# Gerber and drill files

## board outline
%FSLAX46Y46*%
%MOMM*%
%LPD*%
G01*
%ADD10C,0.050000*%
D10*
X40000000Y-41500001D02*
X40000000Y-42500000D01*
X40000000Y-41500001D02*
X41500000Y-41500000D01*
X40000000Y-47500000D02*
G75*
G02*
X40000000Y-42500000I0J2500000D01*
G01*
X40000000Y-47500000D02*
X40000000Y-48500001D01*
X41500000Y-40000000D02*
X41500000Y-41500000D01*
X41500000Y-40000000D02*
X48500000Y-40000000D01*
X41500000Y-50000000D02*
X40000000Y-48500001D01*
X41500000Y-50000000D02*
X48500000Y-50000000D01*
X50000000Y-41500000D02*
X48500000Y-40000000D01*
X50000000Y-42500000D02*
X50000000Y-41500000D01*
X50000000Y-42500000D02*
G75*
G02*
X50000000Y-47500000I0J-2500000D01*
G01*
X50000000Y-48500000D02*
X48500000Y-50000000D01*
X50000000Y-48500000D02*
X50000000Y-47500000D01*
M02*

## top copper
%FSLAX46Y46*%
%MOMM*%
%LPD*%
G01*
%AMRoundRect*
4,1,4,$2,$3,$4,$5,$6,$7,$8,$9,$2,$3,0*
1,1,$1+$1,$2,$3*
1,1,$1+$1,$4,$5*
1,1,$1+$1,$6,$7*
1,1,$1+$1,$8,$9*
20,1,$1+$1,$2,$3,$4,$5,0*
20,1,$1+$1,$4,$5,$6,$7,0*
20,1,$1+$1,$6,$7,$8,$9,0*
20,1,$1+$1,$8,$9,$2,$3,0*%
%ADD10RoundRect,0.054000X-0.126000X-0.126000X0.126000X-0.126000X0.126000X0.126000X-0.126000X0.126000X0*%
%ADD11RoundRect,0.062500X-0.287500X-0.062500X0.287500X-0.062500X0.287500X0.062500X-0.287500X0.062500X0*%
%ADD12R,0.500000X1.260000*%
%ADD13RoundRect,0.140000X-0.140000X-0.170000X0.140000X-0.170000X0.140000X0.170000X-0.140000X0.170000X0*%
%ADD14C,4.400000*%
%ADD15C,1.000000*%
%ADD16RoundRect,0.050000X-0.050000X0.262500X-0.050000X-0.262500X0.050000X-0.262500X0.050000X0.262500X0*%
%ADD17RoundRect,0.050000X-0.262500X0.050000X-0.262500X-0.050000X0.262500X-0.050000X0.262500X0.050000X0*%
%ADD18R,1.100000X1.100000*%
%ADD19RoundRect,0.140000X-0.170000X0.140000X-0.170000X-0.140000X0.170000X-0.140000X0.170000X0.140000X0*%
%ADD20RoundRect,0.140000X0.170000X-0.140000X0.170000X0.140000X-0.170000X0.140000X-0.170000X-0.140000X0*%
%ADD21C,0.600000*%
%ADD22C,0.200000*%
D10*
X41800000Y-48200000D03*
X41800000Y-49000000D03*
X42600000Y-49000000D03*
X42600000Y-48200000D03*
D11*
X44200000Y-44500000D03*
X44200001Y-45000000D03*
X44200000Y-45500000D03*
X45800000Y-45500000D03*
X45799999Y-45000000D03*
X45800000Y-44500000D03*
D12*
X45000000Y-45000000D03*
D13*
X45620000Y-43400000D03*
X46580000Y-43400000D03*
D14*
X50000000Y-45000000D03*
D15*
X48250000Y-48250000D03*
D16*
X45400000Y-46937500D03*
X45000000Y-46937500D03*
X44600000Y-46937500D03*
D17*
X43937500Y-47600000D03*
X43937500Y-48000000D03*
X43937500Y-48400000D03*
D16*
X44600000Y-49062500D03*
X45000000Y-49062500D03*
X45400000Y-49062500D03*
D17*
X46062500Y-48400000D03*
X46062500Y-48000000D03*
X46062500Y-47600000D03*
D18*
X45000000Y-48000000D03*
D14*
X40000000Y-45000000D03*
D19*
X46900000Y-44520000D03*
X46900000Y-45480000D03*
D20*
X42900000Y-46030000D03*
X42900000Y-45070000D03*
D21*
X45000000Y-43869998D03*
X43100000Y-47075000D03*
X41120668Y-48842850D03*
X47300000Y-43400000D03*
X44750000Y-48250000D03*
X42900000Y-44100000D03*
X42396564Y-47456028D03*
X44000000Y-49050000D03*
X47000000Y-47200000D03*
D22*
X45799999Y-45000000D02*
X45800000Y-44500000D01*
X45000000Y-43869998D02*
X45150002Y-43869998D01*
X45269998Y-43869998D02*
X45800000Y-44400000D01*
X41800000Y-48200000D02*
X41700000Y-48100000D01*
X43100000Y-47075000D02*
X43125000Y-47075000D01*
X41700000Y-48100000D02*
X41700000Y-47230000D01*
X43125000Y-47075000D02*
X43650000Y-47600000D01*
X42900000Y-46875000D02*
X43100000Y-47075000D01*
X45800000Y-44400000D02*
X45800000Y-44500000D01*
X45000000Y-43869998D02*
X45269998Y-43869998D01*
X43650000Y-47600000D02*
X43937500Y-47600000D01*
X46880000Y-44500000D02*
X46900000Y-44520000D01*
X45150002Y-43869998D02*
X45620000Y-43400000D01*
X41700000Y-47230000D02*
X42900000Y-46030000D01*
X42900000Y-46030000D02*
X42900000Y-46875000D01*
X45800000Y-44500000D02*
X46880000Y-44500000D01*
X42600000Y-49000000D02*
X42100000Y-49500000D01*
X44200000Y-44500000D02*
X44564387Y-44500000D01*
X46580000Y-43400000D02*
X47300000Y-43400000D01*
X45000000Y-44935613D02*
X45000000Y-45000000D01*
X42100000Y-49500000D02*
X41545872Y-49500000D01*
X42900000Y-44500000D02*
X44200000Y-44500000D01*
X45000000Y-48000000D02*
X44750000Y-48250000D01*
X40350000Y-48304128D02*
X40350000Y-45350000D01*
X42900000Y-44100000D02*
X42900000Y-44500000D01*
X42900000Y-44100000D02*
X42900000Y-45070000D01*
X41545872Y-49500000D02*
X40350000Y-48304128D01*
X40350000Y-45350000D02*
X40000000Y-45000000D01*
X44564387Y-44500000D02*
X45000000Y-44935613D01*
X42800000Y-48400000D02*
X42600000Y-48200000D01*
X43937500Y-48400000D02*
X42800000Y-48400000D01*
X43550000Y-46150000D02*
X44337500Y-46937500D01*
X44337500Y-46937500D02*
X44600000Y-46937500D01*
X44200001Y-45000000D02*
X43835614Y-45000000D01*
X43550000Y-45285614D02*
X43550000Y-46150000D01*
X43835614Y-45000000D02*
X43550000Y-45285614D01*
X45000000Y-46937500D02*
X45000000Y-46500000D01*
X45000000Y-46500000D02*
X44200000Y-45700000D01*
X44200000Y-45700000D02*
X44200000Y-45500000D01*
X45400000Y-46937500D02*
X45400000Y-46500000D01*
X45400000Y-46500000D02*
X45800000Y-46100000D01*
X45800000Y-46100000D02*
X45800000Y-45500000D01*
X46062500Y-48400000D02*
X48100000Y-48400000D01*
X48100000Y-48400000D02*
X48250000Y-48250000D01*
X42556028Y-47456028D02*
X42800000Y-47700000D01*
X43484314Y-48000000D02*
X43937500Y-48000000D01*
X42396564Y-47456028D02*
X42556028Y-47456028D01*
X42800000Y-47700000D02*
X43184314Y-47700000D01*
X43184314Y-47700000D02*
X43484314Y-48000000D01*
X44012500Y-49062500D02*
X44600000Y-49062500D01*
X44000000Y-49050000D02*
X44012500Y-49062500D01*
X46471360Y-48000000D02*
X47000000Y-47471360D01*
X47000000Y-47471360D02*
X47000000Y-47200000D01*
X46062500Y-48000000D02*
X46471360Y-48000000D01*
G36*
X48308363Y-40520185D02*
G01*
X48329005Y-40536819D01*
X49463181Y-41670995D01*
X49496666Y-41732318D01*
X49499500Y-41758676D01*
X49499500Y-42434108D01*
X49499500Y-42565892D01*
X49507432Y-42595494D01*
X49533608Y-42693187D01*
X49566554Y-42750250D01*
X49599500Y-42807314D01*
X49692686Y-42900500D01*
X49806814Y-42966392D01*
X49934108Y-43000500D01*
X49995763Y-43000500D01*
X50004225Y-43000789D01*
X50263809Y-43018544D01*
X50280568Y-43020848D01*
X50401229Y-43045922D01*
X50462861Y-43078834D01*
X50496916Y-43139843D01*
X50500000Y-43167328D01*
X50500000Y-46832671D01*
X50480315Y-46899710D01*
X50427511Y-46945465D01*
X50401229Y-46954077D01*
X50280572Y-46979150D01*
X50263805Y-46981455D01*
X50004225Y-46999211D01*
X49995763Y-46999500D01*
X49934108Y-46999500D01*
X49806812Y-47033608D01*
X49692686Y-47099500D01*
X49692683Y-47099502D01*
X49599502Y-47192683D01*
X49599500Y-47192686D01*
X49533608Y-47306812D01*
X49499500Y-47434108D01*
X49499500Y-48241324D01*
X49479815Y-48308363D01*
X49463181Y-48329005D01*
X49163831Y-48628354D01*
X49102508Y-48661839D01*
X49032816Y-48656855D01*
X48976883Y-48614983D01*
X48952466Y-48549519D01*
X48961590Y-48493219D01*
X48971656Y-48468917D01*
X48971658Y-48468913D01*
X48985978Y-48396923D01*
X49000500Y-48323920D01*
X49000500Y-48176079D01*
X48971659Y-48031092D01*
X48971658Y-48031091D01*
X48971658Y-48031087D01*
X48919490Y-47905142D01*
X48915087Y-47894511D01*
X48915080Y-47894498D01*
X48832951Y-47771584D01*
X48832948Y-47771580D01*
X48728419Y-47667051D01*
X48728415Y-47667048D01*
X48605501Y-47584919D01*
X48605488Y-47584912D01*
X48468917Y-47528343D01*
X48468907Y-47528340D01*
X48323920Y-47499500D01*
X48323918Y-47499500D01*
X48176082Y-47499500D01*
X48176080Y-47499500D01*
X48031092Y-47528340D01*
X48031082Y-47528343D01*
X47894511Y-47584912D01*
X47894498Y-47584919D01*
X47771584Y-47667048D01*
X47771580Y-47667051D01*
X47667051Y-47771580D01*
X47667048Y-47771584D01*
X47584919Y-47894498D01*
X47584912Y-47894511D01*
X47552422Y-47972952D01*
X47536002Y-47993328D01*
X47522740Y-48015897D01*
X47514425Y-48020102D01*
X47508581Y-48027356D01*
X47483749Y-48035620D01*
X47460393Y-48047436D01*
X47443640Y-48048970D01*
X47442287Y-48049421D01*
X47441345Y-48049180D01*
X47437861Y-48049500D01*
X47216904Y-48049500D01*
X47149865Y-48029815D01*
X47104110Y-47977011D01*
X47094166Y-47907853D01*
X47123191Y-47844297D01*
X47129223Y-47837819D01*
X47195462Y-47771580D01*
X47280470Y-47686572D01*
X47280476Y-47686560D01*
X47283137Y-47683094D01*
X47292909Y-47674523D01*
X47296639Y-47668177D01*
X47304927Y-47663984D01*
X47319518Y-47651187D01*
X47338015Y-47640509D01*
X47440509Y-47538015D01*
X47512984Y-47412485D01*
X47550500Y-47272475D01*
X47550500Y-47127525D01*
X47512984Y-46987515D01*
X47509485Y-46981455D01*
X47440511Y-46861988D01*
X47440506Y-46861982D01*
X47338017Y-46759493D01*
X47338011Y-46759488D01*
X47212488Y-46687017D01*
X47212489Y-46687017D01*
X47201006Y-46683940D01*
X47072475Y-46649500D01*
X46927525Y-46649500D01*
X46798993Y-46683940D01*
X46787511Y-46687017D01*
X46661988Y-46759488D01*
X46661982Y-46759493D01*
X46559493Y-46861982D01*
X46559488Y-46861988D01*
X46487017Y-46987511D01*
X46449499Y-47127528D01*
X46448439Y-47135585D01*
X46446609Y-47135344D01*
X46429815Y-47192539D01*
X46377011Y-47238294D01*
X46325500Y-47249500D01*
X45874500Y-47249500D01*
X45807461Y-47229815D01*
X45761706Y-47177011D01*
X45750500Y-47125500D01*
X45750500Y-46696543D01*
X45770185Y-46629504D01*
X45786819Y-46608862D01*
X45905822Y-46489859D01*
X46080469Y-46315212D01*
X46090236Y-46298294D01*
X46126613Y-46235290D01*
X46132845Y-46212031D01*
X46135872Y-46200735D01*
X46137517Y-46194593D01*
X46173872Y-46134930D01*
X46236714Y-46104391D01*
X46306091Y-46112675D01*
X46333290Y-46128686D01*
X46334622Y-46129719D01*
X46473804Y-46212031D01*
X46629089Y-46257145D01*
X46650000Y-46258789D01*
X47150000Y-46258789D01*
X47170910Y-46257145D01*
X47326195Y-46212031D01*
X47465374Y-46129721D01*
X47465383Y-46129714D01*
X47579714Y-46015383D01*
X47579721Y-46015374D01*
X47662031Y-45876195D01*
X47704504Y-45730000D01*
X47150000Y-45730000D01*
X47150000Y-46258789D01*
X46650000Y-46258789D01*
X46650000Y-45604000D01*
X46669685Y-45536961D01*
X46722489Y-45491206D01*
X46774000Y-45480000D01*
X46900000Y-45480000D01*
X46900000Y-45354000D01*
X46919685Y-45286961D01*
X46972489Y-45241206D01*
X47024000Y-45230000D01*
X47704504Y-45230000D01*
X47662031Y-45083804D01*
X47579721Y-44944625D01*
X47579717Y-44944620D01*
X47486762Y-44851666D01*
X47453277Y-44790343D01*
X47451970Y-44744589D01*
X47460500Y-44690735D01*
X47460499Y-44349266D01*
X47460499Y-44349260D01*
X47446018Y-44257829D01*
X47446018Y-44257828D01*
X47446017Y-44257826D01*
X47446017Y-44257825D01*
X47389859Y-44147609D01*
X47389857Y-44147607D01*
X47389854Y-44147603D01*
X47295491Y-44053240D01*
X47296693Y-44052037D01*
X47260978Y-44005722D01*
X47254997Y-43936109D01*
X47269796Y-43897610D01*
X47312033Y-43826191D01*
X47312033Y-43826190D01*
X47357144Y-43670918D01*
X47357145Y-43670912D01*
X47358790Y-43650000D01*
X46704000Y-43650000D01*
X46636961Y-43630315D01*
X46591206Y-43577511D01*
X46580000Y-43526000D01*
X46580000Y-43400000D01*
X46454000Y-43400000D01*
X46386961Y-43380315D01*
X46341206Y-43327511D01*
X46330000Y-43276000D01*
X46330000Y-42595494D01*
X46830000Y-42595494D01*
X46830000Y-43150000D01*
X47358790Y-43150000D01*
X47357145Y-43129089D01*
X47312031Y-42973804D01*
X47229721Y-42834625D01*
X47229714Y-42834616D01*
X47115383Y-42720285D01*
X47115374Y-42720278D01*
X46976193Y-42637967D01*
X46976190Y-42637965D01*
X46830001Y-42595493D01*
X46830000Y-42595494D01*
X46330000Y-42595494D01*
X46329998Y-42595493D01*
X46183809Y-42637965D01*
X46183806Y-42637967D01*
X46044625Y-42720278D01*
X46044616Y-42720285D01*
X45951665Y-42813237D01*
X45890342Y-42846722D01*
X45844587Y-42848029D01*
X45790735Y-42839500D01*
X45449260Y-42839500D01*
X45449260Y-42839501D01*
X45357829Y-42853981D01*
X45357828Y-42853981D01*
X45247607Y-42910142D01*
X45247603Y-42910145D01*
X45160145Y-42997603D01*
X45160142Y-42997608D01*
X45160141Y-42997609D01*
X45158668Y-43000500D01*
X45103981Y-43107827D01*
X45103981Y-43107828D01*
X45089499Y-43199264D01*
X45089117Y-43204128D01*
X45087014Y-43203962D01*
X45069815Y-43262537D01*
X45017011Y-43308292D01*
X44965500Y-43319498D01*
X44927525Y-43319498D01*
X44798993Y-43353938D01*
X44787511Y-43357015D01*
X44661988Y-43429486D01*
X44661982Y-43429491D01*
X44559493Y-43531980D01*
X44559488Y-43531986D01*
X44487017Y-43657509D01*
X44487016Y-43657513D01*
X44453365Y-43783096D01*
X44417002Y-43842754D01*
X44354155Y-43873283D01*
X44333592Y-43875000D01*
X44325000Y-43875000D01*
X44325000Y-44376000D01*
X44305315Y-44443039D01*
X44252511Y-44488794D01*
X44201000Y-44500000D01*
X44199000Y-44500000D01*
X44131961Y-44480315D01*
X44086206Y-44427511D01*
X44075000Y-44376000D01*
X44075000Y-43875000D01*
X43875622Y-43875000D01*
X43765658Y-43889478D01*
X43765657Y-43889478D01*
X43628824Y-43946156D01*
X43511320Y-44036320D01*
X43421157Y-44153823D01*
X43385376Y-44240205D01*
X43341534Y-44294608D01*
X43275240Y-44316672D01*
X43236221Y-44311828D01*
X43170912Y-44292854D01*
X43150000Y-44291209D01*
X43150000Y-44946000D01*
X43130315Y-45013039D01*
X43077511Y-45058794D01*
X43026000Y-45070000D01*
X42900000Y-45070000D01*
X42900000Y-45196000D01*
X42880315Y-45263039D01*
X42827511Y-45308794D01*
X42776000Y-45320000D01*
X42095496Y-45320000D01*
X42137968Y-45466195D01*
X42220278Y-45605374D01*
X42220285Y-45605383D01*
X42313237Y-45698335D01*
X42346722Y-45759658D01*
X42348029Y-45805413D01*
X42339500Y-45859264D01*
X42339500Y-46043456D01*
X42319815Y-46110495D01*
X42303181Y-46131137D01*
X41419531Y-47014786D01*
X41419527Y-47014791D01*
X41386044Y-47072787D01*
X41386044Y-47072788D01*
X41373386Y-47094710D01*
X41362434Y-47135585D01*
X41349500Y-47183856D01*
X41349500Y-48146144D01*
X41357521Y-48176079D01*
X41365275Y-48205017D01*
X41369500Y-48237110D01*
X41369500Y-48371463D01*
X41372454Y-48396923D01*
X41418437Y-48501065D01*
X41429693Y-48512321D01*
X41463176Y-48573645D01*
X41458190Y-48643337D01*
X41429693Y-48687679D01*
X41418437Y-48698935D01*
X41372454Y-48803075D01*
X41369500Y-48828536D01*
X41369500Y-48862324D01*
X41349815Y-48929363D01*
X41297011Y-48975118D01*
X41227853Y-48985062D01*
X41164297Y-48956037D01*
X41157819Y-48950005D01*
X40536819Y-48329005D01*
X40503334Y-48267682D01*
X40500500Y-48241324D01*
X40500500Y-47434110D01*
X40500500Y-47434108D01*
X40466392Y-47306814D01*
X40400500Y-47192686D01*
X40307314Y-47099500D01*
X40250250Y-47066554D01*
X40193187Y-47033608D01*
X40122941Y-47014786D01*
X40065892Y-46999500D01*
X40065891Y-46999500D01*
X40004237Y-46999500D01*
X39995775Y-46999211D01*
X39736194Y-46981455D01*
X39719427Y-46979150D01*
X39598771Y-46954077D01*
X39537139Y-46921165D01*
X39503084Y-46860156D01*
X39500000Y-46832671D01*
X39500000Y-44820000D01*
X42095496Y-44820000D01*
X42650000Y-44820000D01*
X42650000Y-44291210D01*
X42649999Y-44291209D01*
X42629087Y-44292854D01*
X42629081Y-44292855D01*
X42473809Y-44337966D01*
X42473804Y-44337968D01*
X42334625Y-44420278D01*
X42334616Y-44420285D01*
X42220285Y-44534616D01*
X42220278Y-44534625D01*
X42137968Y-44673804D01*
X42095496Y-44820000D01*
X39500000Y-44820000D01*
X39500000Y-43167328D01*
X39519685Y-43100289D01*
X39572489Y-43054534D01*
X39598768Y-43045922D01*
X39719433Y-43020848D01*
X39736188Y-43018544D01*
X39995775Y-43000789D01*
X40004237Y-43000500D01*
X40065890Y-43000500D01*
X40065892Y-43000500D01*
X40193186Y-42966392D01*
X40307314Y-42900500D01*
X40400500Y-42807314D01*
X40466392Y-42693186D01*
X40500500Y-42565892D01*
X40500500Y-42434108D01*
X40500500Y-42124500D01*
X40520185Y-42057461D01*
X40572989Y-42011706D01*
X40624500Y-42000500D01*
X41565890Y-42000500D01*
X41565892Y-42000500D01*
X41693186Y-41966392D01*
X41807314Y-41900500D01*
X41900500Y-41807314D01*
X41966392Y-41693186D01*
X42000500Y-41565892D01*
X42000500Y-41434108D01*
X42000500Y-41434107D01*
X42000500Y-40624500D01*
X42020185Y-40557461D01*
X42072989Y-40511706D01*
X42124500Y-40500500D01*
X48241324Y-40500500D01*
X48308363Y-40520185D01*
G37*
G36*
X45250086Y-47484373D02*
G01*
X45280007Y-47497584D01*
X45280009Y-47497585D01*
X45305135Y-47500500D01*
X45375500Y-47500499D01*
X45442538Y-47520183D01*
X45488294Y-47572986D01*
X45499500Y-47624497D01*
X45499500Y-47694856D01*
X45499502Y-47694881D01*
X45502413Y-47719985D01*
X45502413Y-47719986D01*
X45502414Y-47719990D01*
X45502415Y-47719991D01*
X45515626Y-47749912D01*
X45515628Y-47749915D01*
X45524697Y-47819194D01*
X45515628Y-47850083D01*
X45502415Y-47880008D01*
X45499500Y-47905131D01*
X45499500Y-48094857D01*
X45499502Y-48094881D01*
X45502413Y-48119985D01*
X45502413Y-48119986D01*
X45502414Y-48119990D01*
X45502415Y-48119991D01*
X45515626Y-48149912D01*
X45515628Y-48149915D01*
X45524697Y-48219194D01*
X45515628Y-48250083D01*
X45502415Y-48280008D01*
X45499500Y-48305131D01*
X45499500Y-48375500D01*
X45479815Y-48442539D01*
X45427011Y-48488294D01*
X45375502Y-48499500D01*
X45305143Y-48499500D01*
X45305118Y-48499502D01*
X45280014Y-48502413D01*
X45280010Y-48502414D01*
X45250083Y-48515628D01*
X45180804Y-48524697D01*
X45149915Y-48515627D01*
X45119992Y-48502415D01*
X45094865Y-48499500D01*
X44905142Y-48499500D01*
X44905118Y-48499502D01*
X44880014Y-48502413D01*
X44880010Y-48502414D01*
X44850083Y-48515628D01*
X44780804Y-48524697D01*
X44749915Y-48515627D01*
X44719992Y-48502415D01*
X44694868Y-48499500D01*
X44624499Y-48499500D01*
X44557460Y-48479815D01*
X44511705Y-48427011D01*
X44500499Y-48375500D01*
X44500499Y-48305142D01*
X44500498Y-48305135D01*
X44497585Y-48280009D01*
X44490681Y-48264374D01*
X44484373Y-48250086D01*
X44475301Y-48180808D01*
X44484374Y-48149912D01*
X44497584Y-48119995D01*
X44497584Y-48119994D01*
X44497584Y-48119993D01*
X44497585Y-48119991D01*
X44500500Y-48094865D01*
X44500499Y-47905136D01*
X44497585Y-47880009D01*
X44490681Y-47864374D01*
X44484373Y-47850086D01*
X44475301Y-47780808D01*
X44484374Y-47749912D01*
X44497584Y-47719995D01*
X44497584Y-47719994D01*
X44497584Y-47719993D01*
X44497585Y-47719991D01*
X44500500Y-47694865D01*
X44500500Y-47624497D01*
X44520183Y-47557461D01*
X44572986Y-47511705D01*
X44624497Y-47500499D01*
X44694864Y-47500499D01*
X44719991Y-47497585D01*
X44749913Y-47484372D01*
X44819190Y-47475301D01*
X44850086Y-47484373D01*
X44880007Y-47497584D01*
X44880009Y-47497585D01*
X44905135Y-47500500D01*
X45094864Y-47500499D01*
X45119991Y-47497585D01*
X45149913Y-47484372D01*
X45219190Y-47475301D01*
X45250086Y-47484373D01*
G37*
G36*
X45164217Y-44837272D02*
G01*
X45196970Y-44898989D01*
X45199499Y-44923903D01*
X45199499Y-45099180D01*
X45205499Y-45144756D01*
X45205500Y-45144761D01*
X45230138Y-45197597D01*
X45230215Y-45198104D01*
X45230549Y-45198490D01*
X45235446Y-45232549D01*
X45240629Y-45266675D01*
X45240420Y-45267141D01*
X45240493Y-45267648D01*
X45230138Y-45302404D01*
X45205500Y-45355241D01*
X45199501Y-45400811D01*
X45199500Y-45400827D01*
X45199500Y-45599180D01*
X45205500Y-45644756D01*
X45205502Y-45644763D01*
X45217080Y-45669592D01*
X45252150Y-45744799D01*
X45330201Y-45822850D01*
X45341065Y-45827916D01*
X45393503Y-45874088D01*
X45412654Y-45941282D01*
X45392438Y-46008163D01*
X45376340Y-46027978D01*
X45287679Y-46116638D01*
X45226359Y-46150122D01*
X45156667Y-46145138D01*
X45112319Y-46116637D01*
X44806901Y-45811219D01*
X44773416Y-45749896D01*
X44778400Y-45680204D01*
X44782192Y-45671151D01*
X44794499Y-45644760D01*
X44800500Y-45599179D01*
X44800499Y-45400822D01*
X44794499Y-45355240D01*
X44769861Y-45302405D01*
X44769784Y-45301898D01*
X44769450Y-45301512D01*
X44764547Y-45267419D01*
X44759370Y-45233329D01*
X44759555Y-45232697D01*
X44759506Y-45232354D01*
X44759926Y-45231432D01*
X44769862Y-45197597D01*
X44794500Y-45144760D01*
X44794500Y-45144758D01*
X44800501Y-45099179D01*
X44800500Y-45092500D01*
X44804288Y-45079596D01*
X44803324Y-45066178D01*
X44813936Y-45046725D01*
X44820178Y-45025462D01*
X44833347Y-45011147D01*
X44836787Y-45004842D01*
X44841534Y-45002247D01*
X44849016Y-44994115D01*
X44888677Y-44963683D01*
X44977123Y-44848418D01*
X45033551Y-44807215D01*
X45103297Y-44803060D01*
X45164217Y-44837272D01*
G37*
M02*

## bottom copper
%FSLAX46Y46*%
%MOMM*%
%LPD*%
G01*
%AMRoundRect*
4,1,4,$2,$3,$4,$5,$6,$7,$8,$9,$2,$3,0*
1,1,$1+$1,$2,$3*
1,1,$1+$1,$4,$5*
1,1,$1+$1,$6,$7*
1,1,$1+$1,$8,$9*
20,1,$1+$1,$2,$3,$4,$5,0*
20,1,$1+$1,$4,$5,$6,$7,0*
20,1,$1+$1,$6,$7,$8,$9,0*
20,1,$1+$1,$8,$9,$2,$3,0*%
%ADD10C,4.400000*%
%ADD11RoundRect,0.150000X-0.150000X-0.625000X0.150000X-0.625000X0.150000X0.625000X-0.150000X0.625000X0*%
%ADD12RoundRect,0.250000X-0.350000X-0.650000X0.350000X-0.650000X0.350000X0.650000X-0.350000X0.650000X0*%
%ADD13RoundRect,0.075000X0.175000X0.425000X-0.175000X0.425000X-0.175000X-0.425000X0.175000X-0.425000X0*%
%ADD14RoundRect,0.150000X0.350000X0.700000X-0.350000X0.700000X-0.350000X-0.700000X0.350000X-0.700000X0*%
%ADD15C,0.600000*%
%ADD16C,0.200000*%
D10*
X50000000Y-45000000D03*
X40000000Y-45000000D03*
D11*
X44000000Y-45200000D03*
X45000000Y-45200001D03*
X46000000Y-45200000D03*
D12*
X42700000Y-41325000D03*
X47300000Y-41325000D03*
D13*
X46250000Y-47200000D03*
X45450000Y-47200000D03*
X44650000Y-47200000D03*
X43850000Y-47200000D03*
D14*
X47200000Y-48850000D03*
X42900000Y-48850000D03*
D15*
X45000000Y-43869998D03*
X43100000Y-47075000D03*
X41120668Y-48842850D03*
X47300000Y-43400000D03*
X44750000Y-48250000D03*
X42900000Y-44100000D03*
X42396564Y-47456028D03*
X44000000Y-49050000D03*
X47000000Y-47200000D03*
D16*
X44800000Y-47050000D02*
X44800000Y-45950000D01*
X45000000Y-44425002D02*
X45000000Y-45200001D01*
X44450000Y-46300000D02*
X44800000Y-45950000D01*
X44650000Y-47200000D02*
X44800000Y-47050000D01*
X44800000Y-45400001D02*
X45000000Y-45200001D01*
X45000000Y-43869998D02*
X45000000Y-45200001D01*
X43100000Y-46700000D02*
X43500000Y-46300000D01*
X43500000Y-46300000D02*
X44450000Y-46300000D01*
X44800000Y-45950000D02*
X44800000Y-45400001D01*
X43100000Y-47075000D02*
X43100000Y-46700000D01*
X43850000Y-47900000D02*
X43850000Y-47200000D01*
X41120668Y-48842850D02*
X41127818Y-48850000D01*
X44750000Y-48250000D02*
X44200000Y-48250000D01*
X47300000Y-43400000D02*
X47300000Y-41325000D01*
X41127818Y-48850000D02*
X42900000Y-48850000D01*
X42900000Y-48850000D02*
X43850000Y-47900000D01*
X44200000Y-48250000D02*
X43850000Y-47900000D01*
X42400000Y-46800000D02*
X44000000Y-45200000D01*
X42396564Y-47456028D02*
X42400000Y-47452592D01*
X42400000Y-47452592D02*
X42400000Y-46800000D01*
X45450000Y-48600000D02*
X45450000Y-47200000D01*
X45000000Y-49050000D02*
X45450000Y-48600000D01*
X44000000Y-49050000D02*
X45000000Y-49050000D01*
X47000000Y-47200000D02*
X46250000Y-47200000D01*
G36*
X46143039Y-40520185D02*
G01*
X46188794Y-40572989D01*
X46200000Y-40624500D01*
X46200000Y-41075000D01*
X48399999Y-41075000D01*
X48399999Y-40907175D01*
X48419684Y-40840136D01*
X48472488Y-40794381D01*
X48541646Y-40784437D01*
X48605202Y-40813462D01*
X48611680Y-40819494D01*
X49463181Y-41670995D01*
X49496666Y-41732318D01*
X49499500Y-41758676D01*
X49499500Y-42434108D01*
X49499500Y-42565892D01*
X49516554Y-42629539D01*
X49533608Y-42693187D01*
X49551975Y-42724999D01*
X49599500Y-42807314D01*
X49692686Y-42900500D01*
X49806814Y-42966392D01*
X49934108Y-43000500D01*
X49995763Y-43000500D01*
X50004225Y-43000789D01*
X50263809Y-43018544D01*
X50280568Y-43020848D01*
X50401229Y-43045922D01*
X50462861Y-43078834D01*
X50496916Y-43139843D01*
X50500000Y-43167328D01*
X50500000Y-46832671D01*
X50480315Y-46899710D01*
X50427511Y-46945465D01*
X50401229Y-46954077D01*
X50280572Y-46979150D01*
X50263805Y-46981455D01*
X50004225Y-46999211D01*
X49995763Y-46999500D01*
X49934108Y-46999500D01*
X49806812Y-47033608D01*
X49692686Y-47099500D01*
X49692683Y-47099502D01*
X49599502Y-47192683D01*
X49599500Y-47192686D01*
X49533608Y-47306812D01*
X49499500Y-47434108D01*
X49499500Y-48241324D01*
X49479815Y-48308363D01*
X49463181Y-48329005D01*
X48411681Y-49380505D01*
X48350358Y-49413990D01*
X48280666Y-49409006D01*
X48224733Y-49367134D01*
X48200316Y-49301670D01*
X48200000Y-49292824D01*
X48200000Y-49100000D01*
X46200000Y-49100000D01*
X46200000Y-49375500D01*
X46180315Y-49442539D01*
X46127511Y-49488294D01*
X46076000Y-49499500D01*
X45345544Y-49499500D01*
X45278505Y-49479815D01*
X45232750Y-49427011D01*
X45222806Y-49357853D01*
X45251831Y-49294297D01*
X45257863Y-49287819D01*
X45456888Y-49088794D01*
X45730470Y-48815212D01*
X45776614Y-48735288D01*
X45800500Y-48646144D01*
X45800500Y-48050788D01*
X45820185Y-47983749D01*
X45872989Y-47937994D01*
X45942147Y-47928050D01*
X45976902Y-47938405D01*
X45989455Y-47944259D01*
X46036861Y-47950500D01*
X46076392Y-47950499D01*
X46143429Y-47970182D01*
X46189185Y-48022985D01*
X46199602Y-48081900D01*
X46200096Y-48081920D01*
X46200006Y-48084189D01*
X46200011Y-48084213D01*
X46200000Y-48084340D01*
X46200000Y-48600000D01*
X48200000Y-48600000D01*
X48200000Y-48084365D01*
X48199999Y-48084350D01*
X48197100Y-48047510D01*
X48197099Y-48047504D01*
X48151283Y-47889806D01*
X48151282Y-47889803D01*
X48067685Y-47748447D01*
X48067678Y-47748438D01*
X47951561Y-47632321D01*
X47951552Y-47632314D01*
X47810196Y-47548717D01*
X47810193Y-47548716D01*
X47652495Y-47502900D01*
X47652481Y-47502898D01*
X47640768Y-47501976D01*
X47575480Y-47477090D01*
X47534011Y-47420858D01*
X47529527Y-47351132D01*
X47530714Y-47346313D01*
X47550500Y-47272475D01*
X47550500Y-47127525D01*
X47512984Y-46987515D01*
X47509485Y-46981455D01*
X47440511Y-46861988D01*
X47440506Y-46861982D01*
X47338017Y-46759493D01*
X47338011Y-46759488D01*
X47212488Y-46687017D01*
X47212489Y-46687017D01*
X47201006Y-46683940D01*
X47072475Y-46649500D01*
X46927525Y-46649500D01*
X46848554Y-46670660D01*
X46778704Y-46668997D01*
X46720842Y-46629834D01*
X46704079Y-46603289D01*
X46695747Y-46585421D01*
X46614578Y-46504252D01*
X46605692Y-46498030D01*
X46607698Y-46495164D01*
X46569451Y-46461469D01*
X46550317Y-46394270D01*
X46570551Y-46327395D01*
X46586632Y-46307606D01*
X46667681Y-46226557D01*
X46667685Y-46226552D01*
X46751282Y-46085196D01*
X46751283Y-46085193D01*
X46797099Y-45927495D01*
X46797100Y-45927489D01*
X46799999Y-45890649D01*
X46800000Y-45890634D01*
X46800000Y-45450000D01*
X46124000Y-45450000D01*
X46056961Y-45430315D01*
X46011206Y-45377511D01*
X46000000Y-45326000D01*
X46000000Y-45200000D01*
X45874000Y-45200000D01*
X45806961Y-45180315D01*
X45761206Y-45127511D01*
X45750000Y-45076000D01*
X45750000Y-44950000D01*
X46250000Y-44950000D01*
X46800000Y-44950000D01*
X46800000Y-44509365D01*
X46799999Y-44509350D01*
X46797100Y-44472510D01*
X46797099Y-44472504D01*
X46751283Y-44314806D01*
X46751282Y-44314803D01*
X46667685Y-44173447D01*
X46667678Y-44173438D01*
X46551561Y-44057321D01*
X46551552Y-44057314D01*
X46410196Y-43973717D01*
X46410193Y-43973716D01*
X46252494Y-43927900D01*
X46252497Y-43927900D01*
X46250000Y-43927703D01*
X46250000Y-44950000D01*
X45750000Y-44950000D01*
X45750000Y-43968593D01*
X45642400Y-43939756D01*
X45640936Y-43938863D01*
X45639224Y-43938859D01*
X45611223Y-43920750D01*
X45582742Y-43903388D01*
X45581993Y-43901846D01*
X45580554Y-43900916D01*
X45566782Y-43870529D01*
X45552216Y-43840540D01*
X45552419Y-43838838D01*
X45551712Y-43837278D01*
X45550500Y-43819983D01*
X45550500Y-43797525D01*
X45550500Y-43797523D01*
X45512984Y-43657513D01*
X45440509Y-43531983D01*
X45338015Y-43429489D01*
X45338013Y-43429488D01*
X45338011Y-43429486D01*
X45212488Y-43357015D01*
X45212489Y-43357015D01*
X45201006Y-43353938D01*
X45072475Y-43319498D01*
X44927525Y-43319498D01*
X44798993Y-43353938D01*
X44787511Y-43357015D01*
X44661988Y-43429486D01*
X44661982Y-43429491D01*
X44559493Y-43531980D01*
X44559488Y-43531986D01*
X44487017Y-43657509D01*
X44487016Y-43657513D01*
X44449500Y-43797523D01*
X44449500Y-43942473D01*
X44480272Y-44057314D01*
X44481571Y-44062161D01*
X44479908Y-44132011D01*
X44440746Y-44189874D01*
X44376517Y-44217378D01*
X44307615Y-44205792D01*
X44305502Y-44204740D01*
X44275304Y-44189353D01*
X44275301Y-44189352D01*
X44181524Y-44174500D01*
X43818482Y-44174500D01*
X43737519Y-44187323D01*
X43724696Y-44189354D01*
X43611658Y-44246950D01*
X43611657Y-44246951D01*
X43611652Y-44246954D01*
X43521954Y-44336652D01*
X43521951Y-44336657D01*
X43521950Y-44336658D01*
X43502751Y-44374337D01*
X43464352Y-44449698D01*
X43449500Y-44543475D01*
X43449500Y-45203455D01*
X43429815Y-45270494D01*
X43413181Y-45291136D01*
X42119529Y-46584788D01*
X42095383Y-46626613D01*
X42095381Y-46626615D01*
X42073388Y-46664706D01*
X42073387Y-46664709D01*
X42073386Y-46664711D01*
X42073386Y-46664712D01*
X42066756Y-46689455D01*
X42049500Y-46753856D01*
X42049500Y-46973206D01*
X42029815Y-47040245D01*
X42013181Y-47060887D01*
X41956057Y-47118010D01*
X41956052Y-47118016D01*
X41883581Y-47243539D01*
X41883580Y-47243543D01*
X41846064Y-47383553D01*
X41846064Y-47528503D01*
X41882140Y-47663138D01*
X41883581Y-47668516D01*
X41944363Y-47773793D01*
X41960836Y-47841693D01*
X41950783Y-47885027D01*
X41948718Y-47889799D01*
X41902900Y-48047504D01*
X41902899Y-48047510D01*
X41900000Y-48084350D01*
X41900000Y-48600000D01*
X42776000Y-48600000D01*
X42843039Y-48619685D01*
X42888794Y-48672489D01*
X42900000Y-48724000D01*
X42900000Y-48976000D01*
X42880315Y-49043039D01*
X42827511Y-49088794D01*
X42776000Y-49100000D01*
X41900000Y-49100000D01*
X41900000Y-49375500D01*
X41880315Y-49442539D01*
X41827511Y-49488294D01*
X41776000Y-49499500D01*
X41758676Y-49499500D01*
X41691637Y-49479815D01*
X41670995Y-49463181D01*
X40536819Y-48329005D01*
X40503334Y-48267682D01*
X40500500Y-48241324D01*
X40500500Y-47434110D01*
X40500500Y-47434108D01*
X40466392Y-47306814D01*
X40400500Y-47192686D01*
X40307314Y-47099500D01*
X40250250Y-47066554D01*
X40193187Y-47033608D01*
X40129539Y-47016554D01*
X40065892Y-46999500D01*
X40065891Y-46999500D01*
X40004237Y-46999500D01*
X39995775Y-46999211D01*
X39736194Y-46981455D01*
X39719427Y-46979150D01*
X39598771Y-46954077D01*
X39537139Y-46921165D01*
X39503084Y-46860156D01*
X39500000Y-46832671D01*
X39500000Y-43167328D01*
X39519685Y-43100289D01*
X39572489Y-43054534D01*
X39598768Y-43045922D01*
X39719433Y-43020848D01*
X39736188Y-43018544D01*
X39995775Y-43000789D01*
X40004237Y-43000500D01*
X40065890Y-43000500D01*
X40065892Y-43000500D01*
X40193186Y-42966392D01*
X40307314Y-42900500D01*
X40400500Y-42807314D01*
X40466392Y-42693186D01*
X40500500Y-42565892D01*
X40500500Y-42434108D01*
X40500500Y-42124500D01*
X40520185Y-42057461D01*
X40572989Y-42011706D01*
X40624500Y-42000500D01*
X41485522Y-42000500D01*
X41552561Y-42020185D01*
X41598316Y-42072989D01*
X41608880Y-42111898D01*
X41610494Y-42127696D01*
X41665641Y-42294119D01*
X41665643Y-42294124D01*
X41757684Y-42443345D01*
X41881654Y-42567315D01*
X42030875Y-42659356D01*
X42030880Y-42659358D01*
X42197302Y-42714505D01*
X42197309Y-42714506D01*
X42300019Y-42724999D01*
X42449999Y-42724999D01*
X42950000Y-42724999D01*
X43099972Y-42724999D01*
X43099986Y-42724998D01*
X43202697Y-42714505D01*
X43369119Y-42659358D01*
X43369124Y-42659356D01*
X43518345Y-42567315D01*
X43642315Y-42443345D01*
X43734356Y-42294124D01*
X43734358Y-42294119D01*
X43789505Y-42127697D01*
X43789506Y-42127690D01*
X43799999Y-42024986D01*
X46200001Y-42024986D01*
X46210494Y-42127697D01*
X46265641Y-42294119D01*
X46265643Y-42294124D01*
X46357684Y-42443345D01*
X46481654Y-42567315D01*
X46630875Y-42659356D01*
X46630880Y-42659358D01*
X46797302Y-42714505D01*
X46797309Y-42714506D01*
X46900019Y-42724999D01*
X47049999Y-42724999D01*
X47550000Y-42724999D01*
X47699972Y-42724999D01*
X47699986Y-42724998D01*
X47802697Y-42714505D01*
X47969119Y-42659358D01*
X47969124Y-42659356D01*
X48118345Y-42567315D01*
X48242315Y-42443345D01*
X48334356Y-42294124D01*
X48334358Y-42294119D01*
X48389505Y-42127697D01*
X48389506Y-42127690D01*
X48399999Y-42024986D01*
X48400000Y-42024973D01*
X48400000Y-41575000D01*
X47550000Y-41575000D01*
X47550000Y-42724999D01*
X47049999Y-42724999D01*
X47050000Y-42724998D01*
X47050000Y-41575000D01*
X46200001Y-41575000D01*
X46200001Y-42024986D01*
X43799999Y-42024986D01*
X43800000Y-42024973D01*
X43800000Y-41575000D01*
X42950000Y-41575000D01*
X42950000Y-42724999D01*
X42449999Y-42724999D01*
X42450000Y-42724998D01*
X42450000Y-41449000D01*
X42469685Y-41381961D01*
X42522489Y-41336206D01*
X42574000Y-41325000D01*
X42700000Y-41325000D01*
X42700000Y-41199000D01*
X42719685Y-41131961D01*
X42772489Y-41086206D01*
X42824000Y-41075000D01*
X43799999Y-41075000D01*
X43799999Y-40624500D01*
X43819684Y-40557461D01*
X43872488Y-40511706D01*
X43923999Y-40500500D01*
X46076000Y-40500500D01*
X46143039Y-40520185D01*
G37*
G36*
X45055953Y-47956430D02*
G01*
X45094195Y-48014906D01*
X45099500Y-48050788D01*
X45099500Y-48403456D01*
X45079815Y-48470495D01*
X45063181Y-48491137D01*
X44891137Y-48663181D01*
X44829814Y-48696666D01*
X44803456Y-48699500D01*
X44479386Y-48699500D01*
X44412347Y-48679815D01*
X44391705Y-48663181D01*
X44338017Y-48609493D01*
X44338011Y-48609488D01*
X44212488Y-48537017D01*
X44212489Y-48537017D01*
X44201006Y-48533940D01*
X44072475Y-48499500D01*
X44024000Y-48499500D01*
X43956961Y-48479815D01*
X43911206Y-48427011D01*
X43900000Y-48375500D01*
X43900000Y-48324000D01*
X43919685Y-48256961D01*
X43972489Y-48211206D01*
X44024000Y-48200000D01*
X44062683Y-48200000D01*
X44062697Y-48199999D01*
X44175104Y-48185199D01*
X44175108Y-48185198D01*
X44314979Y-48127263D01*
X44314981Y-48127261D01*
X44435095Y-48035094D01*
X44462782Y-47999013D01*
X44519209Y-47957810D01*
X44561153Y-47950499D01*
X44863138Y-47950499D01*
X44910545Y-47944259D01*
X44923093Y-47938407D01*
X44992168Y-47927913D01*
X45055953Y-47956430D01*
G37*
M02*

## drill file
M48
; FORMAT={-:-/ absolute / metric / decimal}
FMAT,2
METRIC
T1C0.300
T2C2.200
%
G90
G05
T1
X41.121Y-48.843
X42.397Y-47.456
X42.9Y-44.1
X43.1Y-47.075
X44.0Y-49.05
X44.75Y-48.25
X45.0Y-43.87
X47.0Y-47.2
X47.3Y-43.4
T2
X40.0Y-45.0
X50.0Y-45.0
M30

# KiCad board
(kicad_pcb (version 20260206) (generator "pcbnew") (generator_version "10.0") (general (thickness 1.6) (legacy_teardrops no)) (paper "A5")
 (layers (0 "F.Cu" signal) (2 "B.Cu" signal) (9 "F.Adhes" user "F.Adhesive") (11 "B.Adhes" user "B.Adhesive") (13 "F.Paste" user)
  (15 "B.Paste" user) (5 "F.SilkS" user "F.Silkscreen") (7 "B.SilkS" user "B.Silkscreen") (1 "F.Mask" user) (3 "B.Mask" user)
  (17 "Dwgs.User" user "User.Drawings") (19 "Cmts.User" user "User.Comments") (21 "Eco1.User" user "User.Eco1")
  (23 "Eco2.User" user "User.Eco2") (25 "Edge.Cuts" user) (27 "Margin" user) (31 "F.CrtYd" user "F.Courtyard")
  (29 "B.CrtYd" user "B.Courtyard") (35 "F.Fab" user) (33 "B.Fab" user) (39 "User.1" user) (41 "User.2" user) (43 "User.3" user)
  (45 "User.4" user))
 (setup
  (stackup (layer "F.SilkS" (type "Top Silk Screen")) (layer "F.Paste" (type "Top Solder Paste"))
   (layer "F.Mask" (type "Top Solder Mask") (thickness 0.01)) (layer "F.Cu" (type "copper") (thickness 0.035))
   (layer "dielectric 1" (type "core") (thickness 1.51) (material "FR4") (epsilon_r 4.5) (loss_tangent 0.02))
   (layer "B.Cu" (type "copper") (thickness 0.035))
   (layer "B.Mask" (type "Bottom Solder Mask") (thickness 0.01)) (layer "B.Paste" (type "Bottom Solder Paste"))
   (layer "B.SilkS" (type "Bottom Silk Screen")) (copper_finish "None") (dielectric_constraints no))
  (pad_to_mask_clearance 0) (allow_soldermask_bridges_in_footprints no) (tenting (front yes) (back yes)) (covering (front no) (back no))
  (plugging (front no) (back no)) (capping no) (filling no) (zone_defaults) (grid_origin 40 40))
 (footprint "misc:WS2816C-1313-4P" (layer "F.Cu") (at 42.2 48.6)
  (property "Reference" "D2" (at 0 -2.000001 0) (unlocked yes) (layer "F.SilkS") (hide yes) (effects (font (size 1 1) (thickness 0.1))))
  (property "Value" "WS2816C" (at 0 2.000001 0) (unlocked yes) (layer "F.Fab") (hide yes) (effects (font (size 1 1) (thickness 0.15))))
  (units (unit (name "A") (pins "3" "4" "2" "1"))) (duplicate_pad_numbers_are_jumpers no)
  (pad "1" smd roundrect (at -0.4 -0.4) (size 0.36 0.36) (layers "F.Cu" "F.Mask" "F.Paste") (roundrect_rratio 0.15) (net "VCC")
   (solder_mask_margin 0.04) (solder_paste_margin_ratio -0.15))
  (pad "2" smd roundrect (at -0.4 0.4) (size 0.36 0.36) (layers "F.Cu" "F.Mask" "F.Paste") (roundrect_rratio 0.15)
   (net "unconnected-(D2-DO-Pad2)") (solder_mask_margin 0.04) (solder_paste_margin_ratio -0.15))
  (pad "3" smd roundrect (at 0.4 0.4) (size 0.36 0.36) (layers "F.Cu" "F.Mask" "F.Paste") (roundrect_rratio 0.15) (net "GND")
   (solder_mask_margin 0.04) (solder_paste_margin_ratio -0.15))
  (pad "4" smd roundrect (at 0.4 -0.4) (size 0.36 0.36) (layers "F.Cu" "F.Mask" "F.Paste") (roundrect_rratio 0.15) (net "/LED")
   (solder_mask_margin 0.04) (solder_paste_margin_ratio -0.15)))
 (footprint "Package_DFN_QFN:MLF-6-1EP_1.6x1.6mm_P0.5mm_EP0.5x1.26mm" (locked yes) (layer "F.Cu") (at 45 45)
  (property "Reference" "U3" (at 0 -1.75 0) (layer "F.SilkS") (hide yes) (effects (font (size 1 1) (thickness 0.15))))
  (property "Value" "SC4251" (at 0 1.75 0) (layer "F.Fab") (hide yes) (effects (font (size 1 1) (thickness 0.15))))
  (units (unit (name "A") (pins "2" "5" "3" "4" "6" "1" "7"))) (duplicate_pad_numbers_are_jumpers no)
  (pad "" smd roundrect (at 0 -0.315001) (size 0.4 0.51) (layers "F.Paste") (roundrect_rratio 0.25))
  (pad "" smd roundrect (at 0 0.315001) (size 0.4 0.51) (layers "F.Paste") (roundrect_rratio 0.25))
  (pad "1" smd roundrect (at -0.8 -0.5) (size 0.7 0.25) (layers "F.Cu" "F.Mask" "F.Paste") (roundrect_rratio 0.25) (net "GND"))
  (pad "2" smd roundrect (at -0.799999 0) (size 0.7 0.25) (layers "F.Cu" "F.Mask" "F.Paste") (roundrect_rratio 0.25) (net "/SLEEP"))
  (pad "3" smd roundrect (at -0.8 0.5) (size 0.7 0.25) (layers "F.Cu" "F.Mask" "F.Paste") (roundrect_rratio 0.25) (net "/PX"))
  (pad "4" smd roundrect (at 0.8 0.5) (size 0.7 0.25) (layers "F.Cu" "F.Mask" "F.Paste") (roundrect_rratio 0.25) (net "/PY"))
  (pad "5" smd roundrect (at 0.799999 0) (size 0.7 0.25) (layers "F.Cu" "F.Mask" "F.Paste") (roundrect_rratio 0.25) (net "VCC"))
  (pad "6" smd roundrect (at 0.8 -0.5) (size 0.7 0.25) (layers "F.Cu" "F.Mask" "F.Paste") (roundrect_rratio 0.25) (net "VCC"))
  (pad "7" smd rect (at 0 0) (size 0.5 1.26) (layers "F.Cu" "F.Mask") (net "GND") (zone_connect 2)))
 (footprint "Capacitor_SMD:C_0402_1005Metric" (layer "F.Cu") (at 46.1 43.4)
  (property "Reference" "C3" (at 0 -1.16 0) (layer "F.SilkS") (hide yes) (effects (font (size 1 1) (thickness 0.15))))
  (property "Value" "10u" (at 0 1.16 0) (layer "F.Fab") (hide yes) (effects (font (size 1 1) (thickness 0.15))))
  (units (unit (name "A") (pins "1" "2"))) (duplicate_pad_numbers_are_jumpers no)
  (pad "1" smd roundrect (at -0.48 0) (size 0.56 0.62) (layers "F.Cu" "F.Mask" "F.Paste") (roundrect_rratio 0.25) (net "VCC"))
  (pad "2" smd roundrect (at 0.48 0) (size 0.56 0.62) (layers "F.Cu" "F.Mask" "F.Paste") (roundrect_rratio 0.25) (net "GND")))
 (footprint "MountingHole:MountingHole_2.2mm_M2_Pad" (layer "F.Cu") (at 50 45)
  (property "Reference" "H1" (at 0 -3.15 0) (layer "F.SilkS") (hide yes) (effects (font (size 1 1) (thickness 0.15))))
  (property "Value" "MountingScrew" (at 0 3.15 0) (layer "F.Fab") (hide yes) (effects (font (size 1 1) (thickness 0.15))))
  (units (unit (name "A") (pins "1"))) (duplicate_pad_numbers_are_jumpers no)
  (pad "1" thru_hole circle (at 0 0) (size 4.4 4.4) (drill 2.2) (layers "*.Cu" "*.Mask") (remove_unused_layers no) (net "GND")
   (zone_connect 2)))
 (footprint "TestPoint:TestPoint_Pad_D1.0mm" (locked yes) (layer "F.Cu") (at 48.25 48.25)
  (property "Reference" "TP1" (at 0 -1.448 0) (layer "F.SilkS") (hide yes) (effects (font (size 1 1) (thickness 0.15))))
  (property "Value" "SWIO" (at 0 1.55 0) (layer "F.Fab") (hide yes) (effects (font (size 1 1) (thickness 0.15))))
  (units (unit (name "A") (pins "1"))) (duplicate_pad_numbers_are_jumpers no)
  (pad "1" smd circle (at 0 0) (size 1 1) (layers "F.Cu" "F.Mask") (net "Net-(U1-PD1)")))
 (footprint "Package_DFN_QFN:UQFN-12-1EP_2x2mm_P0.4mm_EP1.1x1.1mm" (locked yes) (layer "F.Cu") (at 45 48 -90)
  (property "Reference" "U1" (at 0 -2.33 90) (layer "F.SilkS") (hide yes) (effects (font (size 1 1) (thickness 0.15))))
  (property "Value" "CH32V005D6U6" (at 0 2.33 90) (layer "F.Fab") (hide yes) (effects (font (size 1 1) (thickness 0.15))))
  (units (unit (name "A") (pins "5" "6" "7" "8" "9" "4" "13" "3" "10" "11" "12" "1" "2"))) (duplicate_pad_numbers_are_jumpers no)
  (pad "" smd roundrect (at 0 0 270) (size 0.89 0.89) (layers "F.Paste") (roundrect_rratio 0.25))
  (pad "1" smd roundrect (at -1.0625 -0.4 270) (size 0.625 0.2) (layers "F.Cu" "F.Mask" "F.Paste") (roundrect_rratio 0.25) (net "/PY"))
  (pad "2" smd roundrect (at -1.0625 0 270) (size 0.625 0.2) (layers "F.Cu" "F.Mask" "F.Paste") (roundrect_rratio 0.25) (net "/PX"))
  (pad "3" smd roundrect (at -1.0625 0.4 270) (size 0.625 0.2) (layers "F.Cu" "F.Mask" "F.Paste") (roundrect_rratio 0.25) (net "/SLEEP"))
  (pad "4" smd roundrect (at -0.4 1.0625 270) (size 0.2 0.625) (layers "F.Cu" "F.Mask" "F.Paste") (roundrect_rratio 0.25) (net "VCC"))
  (pad "5" smd roundrect (at 0 1.0625 270) (size 0.2 0.625) (layers "F.Cu" "F.Mask" "F.Paste") (roundrect_rratio 0.25) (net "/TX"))
  (pad "6" smd roundrect (at 0.4 1.0625 270) (size 0.2 0.625) (layers "F.Cu" "F.Mask" "F.Paste") (roundrect_rratio 0.25) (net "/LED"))
  (pad "7" smd roundrect (at 1.0625 0.4 270) (size 0.625 0.2) (layers "F.Cu" "F.Mask" "F.Paste") (roundrect_rratio 0.25) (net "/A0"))
  (pad "8" smd roundrect (at 1.0625 0 270) (size 0.625 0.2) (layers "F.Cu" "F.Mask" "F.Paste") (roundrect_rratio 0.25)
   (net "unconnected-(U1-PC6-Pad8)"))
  (pad "9" smd roundrect (at 1.0625 -0.4 270) (size 0.625 0.2) (layers "F.Cu" "F.Mask" "F.Paste") (roundrect_rratio 0.25)
   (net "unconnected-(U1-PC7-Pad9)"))
  (pad "10" smd roundrect (at 0.4 -1.0625 270) (size 0.2 0.625) (layers "F.Cu" "F.Mask" "F.Paste") (roundrect_rratio 0.25)
   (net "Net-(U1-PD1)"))
  (pad "11" smd roundrect (at 0 -1.0625 270) (size 0.2 0.625) (layers "F.Cu" "F.Mask" "F.Paste") (roundrect_rratio 0.25) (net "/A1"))
  (pad "12" smd roundrect (at -0.4 -1.0625 270) (size 0.2 0.625) (layers "F.Cu" "F.Mask" "F.Paste") (roundrect_rratio 0.25)
   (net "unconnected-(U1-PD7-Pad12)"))
  (pad "13" smd rect (at 0 0 270) (size 1.1 1.1) (layers "F.Cu" "F.Mask") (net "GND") (zone_connect 2)))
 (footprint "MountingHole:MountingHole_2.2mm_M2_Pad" (layer "F.Cu") (at 40 45)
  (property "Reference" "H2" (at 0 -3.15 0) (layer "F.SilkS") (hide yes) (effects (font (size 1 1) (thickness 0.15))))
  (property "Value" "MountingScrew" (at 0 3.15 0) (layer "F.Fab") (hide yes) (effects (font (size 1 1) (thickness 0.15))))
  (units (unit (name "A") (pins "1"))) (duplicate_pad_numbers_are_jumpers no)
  (pad "1" thru_hole circle (at 0 0) (size 4.4 4.4) (drill 2.2) (layers "*.Cu" "*.Mask") (remove_unused_layers no) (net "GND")
   (zone_connect 2)))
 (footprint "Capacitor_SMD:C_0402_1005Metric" (layer "F.Cu") (at 46.9 45 -90)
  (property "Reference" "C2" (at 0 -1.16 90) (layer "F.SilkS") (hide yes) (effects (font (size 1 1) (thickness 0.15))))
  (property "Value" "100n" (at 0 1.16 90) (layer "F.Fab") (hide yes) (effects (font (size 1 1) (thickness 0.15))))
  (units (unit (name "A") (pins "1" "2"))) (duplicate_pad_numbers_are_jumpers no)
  (pad "1" smd roundrect (at -0.48 0 270) (size 0.56 0.62) (layers "F.Cu" "F.Mask" "F.Paste") (roundrect_rratio 0.25) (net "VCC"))
  (pad "2" smd roundrect (at 0.48 0 270) (size 0.56 0.62) (layers "F.Cu" "F.Mask" "F.Paste") (roundrect_rratio 0.25) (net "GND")))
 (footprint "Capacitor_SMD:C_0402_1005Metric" (layer "F.Cu") (at 42.9 45.55 90)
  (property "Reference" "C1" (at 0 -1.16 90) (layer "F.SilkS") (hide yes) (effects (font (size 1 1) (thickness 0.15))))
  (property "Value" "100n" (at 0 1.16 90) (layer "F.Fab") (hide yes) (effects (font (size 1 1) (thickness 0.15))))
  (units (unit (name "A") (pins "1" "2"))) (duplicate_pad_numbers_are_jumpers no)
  (pad "1" smd roundrect (at -0.48 0 90) (size 0.56 0.62) (layers "F.Cu" "F.Mask" "F.Paste") (roundrect_rratio 0.25) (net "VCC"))
  (pad "2" smd roundrect (at 0.48 0 90) (size 0.56 0.62) (layers "F.Cu" "F.Mask" "F.Paste") (roundrect_rratio 0.25) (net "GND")))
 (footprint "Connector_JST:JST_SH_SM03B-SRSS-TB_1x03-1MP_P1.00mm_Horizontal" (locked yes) (layer "B.Cu") (at 45 43.2)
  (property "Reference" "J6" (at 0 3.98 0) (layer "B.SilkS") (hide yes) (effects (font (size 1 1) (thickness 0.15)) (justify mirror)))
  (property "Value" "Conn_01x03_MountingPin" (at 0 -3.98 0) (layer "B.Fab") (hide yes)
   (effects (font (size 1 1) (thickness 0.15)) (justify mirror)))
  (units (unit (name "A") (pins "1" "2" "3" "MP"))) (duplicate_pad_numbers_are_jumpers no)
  (pad "1" smd roundrect (at -1 2) (size 0.6 1.55) (layers "B.Cu" "B.Mask" "B.Paste") (roundrect_rratio 0.25) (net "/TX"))
  (pad "2" smd roundrect (at 0 2.000001) (size 0.6 1.55) (layers "B.Cu" "B.Mask" "B.Paste") (roundrect_rratio 0.25) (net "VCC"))
  (pad "3" smd roundrect (at 1 2) (size 0.6 1.55) (layers "B.Cu" "B.Mask" "B.Paste") (roundrect_rratio 0.25) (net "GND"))
  (pad "MP" smd roundrect (at -2.3 -1.875) (size 1.2 1.8) (layers "B.Cu" "B.Mask" "B.Paste") (roundrect_rratio 0.208333) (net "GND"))
  (pad "MP" smd roundrect (at 2.3 -1.875) (size 1.2 1.8) (layers "B.Cu" "B.Mask" "B.Paste") (roundrect_rratio 0.208333) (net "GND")))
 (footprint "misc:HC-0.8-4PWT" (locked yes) (layer "B.Cu") (at 45.05 48.2 180)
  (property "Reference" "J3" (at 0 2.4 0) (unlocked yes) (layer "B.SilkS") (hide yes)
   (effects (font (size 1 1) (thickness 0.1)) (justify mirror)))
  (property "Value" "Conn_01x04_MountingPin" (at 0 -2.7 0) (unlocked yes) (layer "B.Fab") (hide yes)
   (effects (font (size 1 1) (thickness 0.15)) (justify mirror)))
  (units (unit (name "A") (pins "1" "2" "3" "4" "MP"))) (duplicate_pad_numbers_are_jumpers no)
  (pad "1" smd roundrect (at -1.2 1 180) (size 0.5 1) (layers "B.Cu" "B.Mask" "B.Paste") (roundrect_rratio 0.15) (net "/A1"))
  (pad "2" smd roundrect (at -0.4 1 180) (size 0.5 1) (layers "B.Cu" "B.Mask" "B.Paste") (roundrect_rratio 0.15) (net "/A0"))
  (pad "3" smd roundrect (at 0.4 1 180) (size 0.5 1) (layers "B.Cu" "B.Mask" "B.Paste") (roundrect_rratio 0.15) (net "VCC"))
  (pad "4" smd roundrect (at 1.2 1 180) (size 0.5 1) (layers "B.Cu" "B.Mask" "B.Paste") (roundrect_rratio 0.15) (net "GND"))
  (pad "MP" smd roundrect (at -2.15 -0.65 180) (size 1 1.7) (layers "B.Cu" "B.Mask" "B.Paste") (roundrect_rratio 0.15) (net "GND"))
  (pad "MP" smd roundrect (at 2.15 -0.65 180) (size 1 1.7) (layers "B.Cu" "B.Mask" "B.Paste") (roundrect_rratio 0.15) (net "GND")))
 (gr_line (start 40 41.500001) (end 40 42.5) (stroke (width 0.05) (type default)) (layer "Edge.Cuts"))
 (gr_line (start 40 41.500001) (end 41.5 41.5) (stroke (width 0.05) (type default)) (locked yes) (layer "Edge.Cuts"))
 (gr_arc (start 40 47.5) (mid 37.5 45) (end 40 42.5) (stroke (width 0.05) (type default)) (layer "Edge.Cuts"))
 (gr_line (start 40 47.5) (end 40 48.500001) (stroke (width 0.05) (type default)) (layer "Edge.Cuts"))
 (gr_line (start 41.5 40) (end 41.5 41.5) (stroke (width 0.05) (type default)) (locked yes) (layer "Edge.Cuts"))
 (gr_line (start 41.5 40) (end 48.5 40) (stroke (width 0.05) (type solid)) (locked yes) (layer "Edge.Cuts"))
 (gr_line (start 41.5 50) (end 40 48.500001) (stroke (width 0.05) (type default)) (locked yes) (layer "Edge.Cuts"))
 (gr_line (start 41.5 50) (end 48.5 50) (stroke (width 0.05) (type default)) (locked yes) (layer "Edge.Cuts"))
 (gr_line (start 50 41.5) (end 48.5 40) (stroke (width 0.05) (type default)) (locked yes) (layer "Edge.Cuts"))
 (gr_line (start 50 42.5) (end 50 41.5) (stroke (width 0.05) (type default)) (layer "Edge.Cuts"))
 (gr_arc (start 50 42.5) (mid 52.5 45) (end 50 47.5) (stroke (width 0.05) (type default)) (layer "Edge.Cuts"))
 (gr_line (start 50 48.5) (end 48.5 50) (stroke (width 0.05) (type default)) (locked yes) (layer "Edge.Cuts"))
 (gr_line (start 50 48.5) (end 50 47.5) (stroke (width 0.05) (type default)) (layer "Edge.Cuts"))
 (segment (start 45.799999 45) (end 45.8 44.5) (width 0.2) (layer "F.Cu") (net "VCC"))
 (segment (start 45 43.869998) (end 45.150002 43.869998) (width 0.2) (layer "F.Cu") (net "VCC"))
 (segment (start 45.269998 43.869998) (end 45.8 44.4) (width 0.2) (layer "F.Cu") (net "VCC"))
 (segment (start 41.8 48.2) (end 41.7 48.1) (width 0.2) (layer "F.Cu") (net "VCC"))
 (segment (start 43.1 47.075) (end 43.125 47.075) (width 0.2) (layer "F.Cu") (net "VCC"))
 (segment (start 41.7 48.1) (end 41.7 47.23) (width 0.2) (layer "F.Cu") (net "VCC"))
 (segment (start 43.125 47.075) (end 43.65 47.6) (width 0.2) (layer "F.Cu") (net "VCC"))
 (segment (start 42.9 46.875) (end 43.1 47.075) (width 0.2) (layer "F.Cu") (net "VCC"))
 (segment (start 45.8 44.4) (end 45.8 44.5) (width 0.2) (layer "F.Cu") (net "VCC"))
 (segment (start 45 43.869998) (end 45.269998 43.869998) (width 0.2) (layer "F.Cu") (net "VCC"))
 (segment (start 43.65 47.6) (end 43.9375 47.6) (width 0.2) (layer "F.Cu") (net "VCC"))
 (segment (start 46.88 44.5) (end 46.9 44.52) (width 0.2) (layer "F.Cu") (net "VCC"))
 (segment (start 45.150002 43.869998) (end 45.62 43.4) (width 0.2) (layer "F.Cu") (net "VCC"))
 (segment (start 41.7 47.23) (end 42.9 46.03) (width 0.2) (layer "F.Cu") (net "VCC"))
 (segment (start 42.9 46.03) (end 42.9 46.875) (width 0.2) (layer "F.Cu") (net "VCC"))
 (segment (start 45.8 44.5) (end 46.88 44.5) (width 0.2) (layer "F.Cu") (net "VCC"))
 (via (at 45 43.869998) (size 0.6) (drill 0.3) (layers "F.Cu" "B.Cu") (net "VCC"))
 (via (at 43.1 47.075) (size 0.6) (drill 0.3) (layers "F.Cu" "B.Cu") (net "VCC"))
 (segment (start 44.8 47.05) (end 44.8 45.95) (width 0.2) (layer "B.Cu") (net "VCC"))
 (segment (start 45 44.425002) (end 45 45.200001) (width 0.2) (layer "B.Cu") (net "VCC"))
 (segment (start 44.45 46.3) (end 44.8 45.95) (width 0.2) (layer "B.Cu") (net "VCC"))
 (segment (start 44.65 47.2) (end 44.8 47.05) (width 0.2) (layer "B.Cu") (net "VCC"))
 (segment (start 44.8 45.400001) (end 45 45.200001) (width 0.2) (layer "B.Cu") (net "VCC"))
 (segment (start 45 43.869998) (end 45 45.200001) (width 0.2) (layer "B.Cu") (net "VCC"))
 (segment (start 43.1 46.7) (end 43.5 46.3) (width 0.2) (layer "B.Cu") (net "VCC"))
 (segment (start 43.5 46.3) (end 44.45 46.3) (width 0.2) (layer "B.Cu") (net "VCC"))
 (segment (start 44.8 45.95) (end 44.8 45.400001) (width 0.2) (layer "B.Cu") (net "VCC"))
 (segment (start 43.1 47.075) (end 43.1 46.7) (width 0.2) (layer "B.Cu") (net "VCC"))
 (segment (start 42.6 49) (end 42.1 49.5) (width 0.2) (layer "F.Cu") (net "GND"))
 (segment (start 44.2 44.5) (end 44.564387 44.5) (width 0.2) (layer "F.Cu") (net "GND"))
 (segment (start 46.58 43.4) (end 47.3 43.4) (width 0.2) (layer "F.Cu") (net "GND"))
 (segment (start 45 44.935613) (end 45 45) (width 0.2) (layer "F.Cu") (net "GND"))
 (segment (start 42.1 49.5) (end 41.545872 49.5) (width 0.2) (layer "F.Cu") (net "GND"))
 (segment (start 42.9 44.5) (end 44.2 44.5) (width 0.2) (layer "F.Cu") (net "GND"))
 (segment (start 45 48) (end 44.75 48.25) (width 0.2) (layer "F.Cu") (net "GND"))
 (segment (start 40.35 48.304128) (end 40.35 45.35) (width 0.2) (layer "F.Cu") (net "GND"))
 (segment (start 42.9 44.1) (end 42.9 44.5) (width 0.2) (layer "F.Cu") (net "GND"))
 (segment (start 42.9 44.1) (end 42.9 45.07) (width 0.2) (layer "F.Cu") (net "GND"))
 (segment (start 41.545872 49.5) (end 40.35 48.304128) (width 0.2) (layer "F.Cu") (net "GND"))
 (segment (start 40.35 45.35) (end 40 45) (width 0.2) (layer "F.Cu") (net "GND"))
 (segment (start 44.564387 44.5) (end 45 44.935613) (width 0.2) (layer "F.Cu") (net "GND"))
 (via (at 41.120668 48.84285) (size 0.6) (drill 0.3) (layers "F.Cu" "B.Cu") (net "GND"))
 (via (at 47.3 43.4) (size 0.6) (drill 0.3) (layers "F.Cu" "B.Cu") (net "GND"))
 (via (at 44.75 48.25) (size 0.6) (drill 0.3) (layers "F.Cu" "B.Cu") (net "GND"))
 (via (at 42.9 44.1) (size 0.6) (drill 0.3) (layers "F.Cu" "B.Cu") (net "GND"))
 (segment (start 43.85 47.9) (end 43.85 47.2) (width 0.2) (layer "B.Cu") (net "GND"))
 (segment (start 41.120668 48.84285) (end 41.127818 48.85) (width 0.2) (layer "B.Cu") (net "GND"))
 (segment (start 44.75 48.25) (end 44.2 48.25) (width 0.2) (layer "B.Cu") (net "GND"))
 (segment (start 47.3 43.4) (end 47.3 41.325) (width 0.2) (layer "B.Cu") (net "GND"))
 (segment (start 41.127818 48.85) (end 42.9 48.85) (width 0.2) (layer "B.Cu") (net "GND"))
 (segment (start 42.9 48.85) (end 43.85 47.9) (width 0.2) (layer "B.Cu") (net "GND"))
 (segment (start 44.2 48.25) (end 43.85 47.9) (width 0.2) (layer "B.Cu") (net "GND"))
 (segment (start 42.8 48.4) (end 42.6 48.2) (width 0.2) (layer "F.Cu") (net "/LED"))
 (segment (start 43.9375 48.4) (end 42.8 48.4) (width 0.2) (layer "F.Cu") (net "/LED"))
 (segment (start 43.55 46.15) (end 44.3375 46.9375) (width 0.2) (layer "F.Cu") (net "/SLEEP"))
 (segment (start 44.3375 46.9375) (end 44.6 46.9375) (width 0.2) (layer "F.Cu") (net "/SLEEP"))
 (segment (start 44.200001 45) (end 43.835614 45) (width 0.2) (layer "F.Cu") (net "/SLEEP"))
 (segment (start 43.55 45.285614) (end 43.55 46.15) (width 0.2) (layer "F.Cu") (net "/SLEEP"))
 (segment (start 43.835614 45) (end 43.55 45.285614) (width 0.2) (layer "F.Cu") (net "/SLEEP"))
 (segment (start 45 46.9375) (end 45 46.5) (width 0.2) (layer "F.Cu") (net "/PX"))
 (segment (start 45 46.5) (end 44.2 45.7) (width 0.2) (layer "F.Cu") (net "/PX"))
 (segment (start 44.2 45.7) (end 44.2 45.5) (width 0.2) (layer "F.Cu") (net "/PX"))
 (segment (start 45.4 46.9375) (end 45.4 46.5) (width 0.2) (layer "F.Cu") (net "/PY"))
 (segment (start 45.4 46.5) (end 45.8 46.1) (width 0.2) (layer "F.Cu") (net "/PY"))
 (segment (start 45.8 46.1) (end 45.8 45.5) (width 0.2) (layer "F.Cu") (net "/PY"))
 (segment (start 46.0625 48.4) (end 48.1 48.4) (width 0.2) (layer "F.Cu") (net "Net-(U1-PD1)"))
 (segment (start 48.1 48.4) (end 48.25 48.25) (width 0.2) (layer "F.Cu") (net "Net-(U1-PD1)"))
 (segment (start 42.556028 47.456028) (end 42.8 47.7) (width 0.2) (layer "F.Cu") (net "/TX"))
 (segment (start 43.484314 48) (end 43.9375 48) (width 0.2) (layer "F.Cu") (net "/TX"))
 (segment (start 42.396564 47.456028) (end 42.556028 47.456028) (width 0.2) (layer "F.Cu") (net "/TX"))
 (segment (start 42.8 47.7) (end 43.184314 47.7) (width 0.2) (layer "F.Cu") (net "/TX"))
 (segment (start 43.184314 47.7) (end 43.484314 48) (width 0.2) (layer "F.Cu") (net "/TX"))
 (via (at 42.396564 47.456028) (size 0.6) (drill 0.3) (layers "F.Cu" "B.Cu") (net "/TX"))
 (segment (start 42.4 46.8) (end 44 45.2) (width 0.2) (layer "B.Cu") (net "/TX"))
 (segment (start 42.396564 47.456028) (end 42.4 47.452592) (width 0.2) (layer "B.Cu") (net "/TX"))
 (segment (start 42.4 47.452592) (end 42.4 46.8) (width 0.2) (layer "B.Cu") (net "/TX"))
 (segment (start 44.0125 49.0625) (end 44.6 49.0625) (width 0.2) (layer "F.Cu") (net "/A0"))
 (segment (start 44 49.05) (end 44.0125 49.0625) (width 0.2) (layer "F.Cu") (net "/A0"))
 (via (at 44 49.05) (size 0.6) (drill 0.3) (layers "F.Cu" "B.Cu") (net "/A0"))
 (segment (start 45.45 48.6) (end 45.45 47.2) (width 0.2) (layer "B.Cu") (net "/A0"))
 (segment (start 45 49.05) (end 45.45 48.6) (width 0.2) (layer "B.Cu") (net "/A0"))
 (segment (start 44 49.05) (end 45 49.05) (width 0.2) (layer "B.Cu") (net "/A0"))
 (segment (start 46.47136 48) (end 47 47.47136) (width 0.2) (layer "F.Cu") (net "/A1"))
 (segment (start 47 47.47136) (end 47 47.2) (width 0.2) (layer "F.Cu") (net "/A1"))
 (segment (start 46.0625 48) (end 46.47136 48) (width 0.2) (layer "F.Cu") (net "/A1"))
 (via (at 47 47.2) (size 0.6) (drill 0.3) (layers "F.Cu" "B.Cu") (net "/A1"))
 (segment (start 47 47.2) (end 46.25 47.2) (width 0.2) (layer "B.Cu") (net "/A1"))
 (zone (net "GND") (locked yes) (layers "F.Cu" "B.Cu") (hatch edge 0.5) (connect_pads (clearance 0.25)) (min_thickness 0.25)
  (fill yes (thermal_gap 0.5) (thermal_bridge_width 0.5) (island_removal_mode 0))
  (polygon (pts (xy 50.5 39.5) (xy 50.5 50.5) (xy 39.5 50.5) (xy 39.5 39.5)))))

